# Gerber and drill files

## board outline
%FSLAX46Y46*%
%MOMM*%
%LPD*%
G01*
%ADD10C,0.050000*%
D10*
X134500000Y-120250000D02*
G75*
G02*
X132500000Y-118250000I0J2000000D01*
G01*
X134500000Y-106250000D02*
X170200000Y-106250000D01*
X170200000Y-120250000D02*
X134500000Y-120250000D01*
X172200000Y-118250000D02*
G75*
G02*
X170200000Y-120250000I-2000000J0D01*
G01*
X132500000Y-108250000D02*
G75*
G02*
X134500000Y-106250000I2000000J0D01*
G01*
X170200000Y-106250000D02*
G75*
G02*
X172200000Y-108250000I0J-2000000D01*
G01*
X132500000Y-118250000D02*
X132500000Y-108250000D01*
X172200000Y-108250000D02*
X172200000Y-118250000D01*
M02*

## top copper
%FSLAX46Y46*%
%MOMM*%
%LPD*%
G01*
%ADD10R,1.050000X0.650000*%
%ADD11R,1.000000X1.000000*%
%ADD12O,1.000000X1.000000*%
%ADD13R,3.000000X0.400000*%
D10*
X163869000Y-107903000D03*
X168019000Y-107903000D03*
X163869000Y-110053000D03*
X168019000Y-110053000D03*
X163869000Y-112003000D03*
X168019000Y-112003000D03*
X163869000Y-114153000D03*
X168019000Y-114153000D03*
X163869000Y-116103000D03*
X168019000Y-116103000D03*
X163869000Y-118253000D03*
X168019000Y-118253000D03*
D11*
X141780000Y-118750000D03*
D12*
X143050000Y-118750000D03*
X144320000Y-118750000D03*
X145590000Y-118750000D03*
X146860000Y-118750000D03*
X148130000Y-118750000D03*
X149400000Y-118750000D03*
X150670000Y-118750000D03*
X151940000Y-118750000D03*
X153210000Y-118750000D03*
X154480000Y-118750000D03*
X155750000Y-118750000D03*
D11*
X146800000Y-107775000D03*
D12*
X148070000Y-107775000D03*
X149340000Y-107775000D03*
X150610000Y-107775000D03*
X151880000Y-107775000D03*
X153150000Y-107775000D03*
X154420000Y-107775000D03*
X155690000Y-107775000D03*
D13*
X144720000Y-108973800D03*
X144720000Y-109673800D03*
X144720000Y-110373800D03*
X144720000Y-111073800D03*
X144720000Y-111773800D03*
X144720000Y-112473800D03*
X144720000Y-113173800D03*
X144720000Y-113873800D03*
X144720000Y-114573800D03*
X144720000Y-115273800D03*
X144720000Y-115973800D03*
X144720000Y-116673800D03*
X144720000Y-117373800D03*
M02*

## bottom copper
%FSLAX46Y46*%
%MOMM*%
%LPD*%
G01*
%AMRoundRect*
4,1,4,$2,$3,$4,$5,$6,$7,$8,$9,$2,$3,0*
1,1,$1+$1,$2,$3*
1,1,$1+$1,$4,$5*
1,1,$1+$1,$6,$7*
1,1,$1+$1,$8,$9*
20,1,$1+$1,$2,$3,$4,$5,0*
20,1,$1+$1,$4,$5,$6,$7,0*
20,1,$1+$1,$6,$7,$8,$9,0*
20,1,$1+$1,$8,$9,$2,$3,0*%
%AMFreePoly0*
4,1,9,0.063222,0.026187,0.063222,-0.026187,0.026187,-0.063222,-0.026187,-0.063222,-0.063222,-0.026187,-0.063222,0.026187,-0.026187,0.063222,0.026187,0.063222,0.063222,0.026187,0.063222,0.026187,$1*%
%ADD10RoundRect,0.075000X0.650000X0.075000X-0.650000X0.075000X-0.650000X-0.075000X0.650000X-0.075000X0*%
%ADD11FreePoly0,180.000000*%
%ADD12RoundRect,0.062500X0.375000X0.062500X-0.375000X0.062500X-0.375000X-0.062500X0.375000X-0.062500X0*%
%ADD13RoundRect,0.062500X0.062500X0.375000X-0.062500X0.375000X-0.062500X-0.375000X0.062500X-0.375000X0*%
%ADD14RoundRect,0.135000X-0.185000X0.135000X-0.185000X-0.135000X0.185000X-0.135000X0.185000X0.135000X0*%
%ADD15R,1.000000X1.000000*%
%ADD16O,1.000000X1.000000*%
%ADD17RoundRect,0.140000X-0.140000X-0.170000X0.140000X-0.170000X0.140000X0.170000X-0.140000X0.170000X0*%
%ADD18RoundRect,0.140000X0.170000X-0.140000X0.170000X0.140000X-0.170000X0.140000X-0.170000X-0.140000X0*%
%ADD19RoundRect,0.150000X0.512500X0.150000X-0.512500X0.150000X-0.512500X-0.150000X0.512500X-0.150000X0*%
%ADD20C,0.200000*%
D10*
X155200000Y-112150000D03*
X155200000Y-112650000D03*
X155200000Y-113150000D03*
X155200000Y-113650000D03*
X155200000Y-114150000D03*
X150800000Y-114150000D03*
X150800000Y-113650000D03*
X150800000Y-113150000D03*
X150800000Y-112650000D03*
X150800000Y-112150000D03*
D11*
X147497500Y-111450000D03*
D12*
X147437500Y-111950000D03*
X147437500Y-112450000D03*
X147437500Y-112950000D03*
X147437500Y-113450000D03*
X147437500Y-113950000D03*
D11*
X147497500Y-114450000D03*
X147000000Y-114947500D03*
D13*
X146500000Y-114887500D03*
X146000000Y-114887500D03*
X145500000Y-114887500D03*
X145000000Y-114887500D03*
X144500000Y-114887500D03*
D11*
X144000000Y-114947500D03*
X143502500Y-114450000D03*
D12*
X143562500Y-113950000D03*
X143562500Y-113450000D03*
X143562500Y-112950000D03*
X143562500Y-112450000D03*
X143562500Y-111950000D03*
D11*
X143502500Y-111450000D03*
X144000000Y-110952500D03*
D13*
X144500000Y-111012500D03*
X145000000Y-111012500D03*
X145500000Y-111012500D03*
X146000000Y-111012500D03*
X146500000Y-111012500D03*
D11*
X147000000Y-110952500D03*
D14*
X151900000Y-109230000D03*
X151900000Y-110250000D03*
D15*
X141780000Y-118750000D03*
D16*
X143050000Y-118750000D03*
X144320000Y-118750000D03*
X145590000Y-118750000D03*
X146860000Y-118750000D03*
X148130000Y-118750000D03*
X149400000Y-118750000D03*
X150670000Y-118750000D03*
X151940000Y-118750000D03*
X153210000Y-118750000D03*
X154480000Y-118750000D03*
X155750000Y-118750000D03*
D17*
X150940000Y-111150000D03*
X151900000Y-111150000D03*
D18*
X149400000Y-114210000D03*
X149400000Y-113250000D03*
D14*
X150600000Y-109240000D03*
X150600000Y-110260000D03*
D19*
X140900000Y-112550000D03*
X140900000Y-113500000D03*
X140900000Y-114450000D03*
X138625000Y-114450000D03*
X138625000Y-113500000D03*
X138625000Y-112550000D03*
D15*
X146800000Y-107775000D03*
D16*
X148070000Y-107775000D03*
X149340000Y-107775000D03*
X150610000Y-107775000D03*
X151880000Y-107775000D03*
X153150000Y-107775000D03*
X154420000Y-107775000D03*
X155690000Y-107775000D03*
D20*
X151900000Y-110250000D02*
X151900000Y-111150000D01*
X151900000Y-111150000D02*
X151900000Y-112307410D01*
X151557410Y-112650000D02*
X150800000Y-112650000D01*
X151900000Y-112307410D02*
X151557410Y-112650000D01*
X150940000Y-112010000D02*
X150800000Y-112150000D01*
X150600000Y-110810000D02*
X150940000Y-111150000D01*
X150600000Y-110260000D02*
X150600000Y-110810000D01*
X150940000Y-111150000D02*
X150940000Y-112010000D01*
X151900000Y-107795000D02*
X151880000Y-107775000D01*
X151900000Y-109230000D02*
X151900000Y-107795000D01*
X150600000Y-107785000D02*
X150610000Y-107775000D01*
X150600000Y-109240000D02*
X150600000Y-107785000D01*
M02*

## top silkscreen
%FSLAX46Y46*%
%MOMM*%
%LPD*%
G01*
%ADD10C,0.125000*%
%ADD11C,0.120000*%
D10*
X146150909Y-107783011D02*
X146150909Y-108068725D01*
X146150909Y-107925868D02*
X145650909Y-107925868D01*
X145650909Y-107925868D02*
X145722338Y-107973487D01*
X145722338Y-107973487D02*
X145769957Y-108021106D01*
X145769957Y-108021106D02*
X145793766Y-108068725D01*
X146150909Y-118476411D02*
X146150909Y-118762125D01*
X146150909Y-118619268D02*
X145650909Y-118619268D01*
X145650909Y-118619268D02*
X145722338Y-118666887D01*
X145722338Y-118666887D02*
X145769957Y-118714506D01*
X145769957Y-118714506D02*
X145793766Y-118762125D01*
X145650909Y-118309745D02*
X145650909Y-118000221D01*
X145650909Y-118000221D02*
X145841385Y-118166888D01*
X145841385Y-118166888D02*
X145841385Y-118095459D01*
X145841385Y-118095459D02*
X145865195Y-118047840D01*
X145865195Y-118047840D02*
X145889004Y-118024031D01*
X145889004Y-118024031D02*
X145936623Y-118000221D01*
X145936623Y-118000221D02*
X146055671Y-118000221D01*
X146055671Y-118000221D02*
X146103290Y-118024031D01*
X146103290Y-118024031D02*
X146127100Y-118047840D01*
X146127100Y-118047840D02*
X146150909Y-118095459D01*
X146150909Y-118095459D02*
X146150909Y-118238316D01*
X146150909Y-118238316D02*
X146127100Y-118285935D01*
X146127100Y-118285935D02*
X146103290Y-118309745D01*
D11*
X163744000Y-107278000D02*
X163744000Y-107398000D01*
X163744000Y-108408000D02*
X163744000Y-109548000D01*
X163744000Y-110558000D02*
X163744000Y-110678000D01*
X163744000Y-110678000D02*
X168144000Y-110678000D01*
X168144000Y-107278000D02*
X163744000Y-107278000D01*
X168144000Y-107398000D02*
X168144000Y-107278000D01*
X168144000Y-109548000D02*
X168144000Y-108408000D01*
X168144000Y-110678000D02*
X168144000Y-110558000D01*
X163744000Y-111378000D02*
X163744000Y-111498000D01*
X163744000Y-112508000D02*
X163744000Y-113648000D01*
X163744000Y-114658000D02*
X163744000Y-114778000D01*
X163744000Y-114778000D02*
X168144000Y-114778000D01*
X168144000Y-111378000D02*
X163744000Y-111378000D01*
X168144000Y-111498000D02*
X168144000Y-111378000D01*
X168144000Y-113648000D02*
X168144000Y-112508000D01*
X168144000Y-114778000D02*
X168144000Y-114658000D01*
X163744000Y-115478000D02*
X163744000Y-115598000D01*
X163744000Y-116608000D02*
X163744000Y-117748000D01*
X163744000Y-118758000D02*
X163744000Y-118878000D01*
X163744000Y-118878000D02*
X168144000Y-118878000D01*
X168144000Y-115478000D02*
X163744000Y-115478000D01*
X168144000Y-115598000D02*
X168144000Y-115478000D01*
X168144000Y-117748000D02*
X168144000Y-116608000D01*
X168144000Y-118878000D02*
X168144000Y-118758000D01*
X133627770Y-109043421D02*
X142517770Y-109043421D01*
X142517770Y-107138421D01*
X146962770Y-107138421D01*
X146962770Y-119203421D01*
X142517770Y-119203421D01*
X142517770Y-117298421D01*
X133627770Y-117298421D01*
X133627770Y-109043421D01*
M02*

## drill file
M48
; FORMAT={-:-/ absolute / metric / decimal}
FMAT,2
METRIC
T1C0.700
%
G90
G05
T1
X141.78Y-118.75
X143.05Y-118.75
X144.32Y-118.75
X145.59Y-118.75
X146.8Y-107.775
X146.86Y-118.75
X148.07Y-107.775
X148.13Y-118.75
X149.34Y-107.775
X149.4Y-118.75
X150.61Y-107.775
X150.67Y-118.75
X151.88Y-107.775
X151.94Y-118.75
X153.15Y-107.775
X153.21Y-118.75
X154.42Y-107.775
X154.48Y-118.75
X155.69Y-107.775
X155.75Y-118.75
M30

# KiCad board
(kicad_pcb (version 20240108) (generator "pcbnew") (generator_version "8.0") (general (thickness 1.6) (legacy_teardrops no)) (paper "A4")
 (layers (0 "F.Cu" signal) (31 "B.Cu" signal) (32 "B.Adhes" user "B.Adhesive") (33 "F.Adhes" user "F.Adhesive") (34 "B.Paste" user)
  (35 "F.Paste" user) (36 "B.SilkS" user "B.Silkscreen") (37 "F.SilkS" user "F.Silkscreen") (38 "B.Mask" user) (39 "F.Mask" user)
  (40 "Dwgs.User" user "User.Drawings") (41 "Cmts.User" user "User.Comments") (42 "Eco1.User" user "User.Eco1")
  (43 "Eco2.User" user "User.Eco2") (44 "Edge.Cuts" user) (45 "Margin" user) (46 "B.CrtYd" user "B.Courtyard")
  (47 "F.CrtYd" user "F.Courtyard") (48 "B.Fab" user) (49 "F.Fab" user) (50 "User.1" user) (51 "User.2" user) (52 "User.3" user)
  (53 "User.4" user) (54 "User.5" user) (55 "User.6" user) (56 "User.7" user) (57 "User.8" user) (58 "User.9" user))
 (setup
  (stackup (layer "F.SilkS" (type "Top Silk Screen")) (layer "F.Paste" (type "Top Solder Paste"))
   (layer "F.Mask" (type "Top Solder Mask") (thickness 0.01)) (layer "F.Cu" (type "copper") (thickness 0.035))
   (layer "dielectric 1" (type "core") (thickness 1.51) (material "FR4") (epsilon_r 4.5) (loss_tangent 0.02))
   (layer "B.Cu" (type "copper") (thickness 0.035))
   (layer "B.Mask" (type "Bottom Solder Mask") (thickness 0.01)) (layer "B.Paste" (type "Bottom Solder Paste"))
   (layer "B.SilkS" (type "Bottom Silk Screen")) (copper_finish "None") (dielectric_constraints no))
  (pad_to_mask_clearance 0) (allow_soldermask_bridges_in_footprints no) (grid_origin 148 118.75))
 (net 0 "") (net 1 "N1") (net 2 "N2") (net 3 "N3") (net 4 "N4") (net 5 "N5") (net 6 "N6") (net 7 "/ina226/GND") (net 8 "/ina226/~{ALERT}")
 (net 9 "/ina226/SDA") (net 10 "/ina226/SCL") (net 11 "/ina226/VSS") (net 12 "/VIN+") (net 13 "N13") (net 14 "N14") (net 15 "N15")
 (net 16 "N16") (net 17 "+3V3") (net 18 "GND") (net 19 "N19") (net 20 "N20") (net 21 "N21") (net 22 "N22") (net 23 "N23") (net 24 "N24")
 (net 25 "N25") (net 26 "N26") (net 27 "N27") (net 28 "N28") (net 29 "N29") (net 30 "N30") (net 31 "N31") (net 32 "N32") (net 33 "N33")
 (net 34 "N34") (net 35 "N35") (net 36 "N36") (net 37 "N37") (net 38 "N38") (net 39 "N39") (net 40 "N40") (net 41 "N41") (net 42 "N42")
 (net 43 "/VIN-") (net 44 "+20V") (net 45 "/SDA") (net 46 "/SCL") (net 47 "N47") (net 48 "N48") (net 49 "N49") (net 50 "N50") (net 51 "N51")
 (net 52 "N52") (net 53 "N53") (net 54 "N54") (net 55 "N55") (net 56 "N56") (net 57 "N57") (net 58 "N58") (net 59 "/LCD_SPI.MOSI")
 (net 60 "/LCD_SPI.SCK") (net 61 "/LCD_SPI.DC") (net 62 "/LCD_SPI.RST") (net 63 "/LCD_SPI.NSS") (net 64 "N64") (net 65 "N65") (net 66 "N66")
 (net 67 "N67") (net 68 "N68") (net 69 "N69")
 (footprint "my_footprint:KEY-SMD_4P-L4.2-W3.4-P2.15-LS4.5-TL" (layer "F.Cu") (at 166 109.05)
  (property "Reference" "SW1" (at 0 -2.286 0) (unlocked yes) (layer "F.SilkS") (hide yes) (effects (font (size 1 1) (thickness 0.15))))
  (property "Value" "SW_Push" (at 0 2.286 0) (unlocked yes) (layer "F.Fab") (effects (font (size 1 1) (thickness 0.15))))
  (fp_line (start -2.256 -1.772) (end -2.256 -1.652) (stroke (width 0.12) (type solid)) (layer "F.SilkS"))
  (fp_line (start -2.256 -0.642) (end -2.256 0.498) (stroke (width 0.12) (type solid)) (layer "F.SilkS"))
  (fp_line (start -2.256 1.508) (end -2.256 1.628) (stroke (width 0.12) (type solid)) (layer "F.SilkS"))
  (fp_line (start -2.256 1.628) (end 2.144 1.628) (stroke (width 0.12) (type solid)) (layer "F.SilkS"))
  (fp_line (start 2.144 -1.772) (end -2.256 -1.772) (stroke (width 0.12) (type solid)) (layer "F.SilkS"))
  (fp_line (start 2.144 -1.652) (end 2.144 -1.772) (stroke (width 0.12) (type solid)) (layer "F.SilkS"))
  (fp_line (start 2.144 0.498) (end 2.144 -0.642) (stroke (width 0.12) (type solid)) (layer "F.SilkS"))
  (fp_line (start 2.144 1.628) (end 2.144 1.508) (stroke (width 0.12) (type solid)) (layer "F.SilkS"))
  (pad "1" smd rect (at -2.131 -1.147) (size 1.05 0.65) (layers "F.Cu" "F.Paste" "F.Mask") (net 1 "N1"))
  (pad "1" smd rect (at 2.019 -1.147) (size 1.05 0.65) (layers "F.Cu" "F.Paste" "F.Mask") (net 1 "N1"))
  (pad "2" smd rect (at -2.131 1.003) (size 1.05 0.65) (layers "F.Cu" "F.Paste" "F.Mask") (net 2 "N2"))
  (pad "2" smd rect (at 2.019 1.003) (size 1.05 0.65) (layers "F.Cu" "F.Paste" "F.Mask") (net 2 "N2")))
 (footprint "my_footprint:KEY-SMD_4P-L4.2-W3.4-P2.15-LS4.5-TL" (layer "F.Cu") (at 166 113.15)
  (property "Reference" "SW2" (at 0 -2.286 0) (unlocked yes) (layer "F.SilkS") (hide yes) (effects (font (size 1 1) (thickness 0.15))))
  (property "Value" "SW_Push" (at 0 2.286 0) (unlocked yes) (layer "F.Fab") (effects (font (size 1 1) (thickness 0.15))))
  (fp_line (start -2.256 -1.772) (end -2.256 -1.652) (stroke (width 0.12) (type solid)) (layer "F.SilkS"))
  (fp_line (start -2.256 -0.642) (end -2.256 0.498) (stroke (width 0.12) (type solid)) (layer "F.SilkS"))
  (fp_line (start -2.256 1.508) (end -2.256 1.628) (stroke (width 0.12) (type solid)) (layer "F.SilkS"))
  (fp_line (start -2.256 1.628) (end 2.144 1.628) (stroke (width 0.12) (type solid)) (layer "F.SilkS"))
  (fp_line (start 2.144 -1.772) (end -2.256 -1.772) (stroke (width 0.12) (type solid)) (layer "F.SilkS"))
  (fp_line (start 2.144 -1.652) (end 2.144 -1.772) (stroke (width 0.12) (type solid)) (layer "F.SilkS"))
  (fp_line (start 2.144 0.498) (end 2.144 -0.642) (stroke (width 0.12) (type solid)) (layer "F.SilkS"))
  (fp_line (start 2.144 1.628) (end 2.144 1.508) (stroke (width 0.12) (type solid)) (layer "F.SilkS"))
  (pad "1" smd rect (at -2.131 -1.147) (size 1.05 0.65) (layers "F.Cu" "F.Paste" "F.Mask") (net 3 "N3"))
  (pad "1" smd rect (at 2.019 -1.147) (size 1.05 0.65) (layers "F.Cu" "F.Paste" "F.Mask") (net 3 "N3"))
  (pad "2" smd rect (at -2.131 1.003) (size 1.05 0.65) (layers "F.Cu" "F.Paste" "F.Mask") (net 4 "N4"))
  (pad "2" smd rect (at 2.019 1.003) (size 1.05 0.65) (layers "F.Cu" "F.Paste" "F.Mask") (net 4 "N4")))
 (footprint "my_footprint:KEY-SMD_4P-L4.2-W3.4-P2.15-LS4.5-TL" (layer "F.Cu") (at 166 117.25)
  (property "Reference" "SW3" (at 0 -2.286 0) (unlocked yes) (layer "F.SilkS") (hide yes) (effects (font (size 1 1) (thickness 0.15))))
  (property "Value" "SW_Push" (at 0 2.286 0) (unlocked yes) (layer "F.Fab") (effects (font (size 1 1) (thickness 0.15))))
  (fp_line (start -2.256 -1.772) (end -2.256 -1.652) (stroke (width 0.12) (type solid)) (layer "F.SilkS"))
  (fp_line (start -2.256 -0.642) (end -2.256 0.498) (stroke (width 0.12) (type solid)) (layer "F.SilkS"))
  (fp_line (start -2.256 1.508) (end -2.256 1.628) (stroke (width 0.12) (type solid)) (layer "F.SilkS"))
  (fp_line (start -2.256 1.628) (end 2.144 1.628) (stroke (width 0.12) (type solid)) (layer "F.SilkS"))
  (fp_line (start 2.144 -1.772) (end -2.256 -1.772) (stroke (width 0.12) (type solid)) (layer "F.SilkS"))
  (fp_line (start 2.144 -1.652) (end 2.144 -1.772) (stroke (width 0.12) (type solid)) (layer "F.SilkS"))
  (fp_line (start 2.144 0.498) (end 2.144 -0.642) (stroke (width 0.12) (type solid)) (layer "F.SilkS"))
  (fp_line (start 2.144 1.628) (end 2.144 1.508) (stroke (width 0.12) (type solid)) (layer "F.SilkS"))
  (pad "1" smd rect (at -2.131 -1.147) (size 1.05 0.65) (layers "F.Cu" "F.Paste" "F.Mask") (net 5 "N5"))
  (pad "1" smd rect (at 2.019 -1.147) (size 1.05 0.65) (layers "F.Cu" "F.Paste" "F.Mask") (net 5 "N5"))
  (pad "2" smd rect (at -2.131 1.003) (size 1.05 0.65) (layers "F.Cu" "F.Paste" "F.Mask") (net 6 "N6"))
  (pad "2" smd rect (at 2.019 1.003) (size 1.05 0.65) (layers "F.Cu" "F.Paste" "F.Mask") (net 6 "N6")))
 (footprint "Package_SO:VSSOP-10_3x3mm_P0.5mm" (layer "B.Cu") (at 153 113.15 180)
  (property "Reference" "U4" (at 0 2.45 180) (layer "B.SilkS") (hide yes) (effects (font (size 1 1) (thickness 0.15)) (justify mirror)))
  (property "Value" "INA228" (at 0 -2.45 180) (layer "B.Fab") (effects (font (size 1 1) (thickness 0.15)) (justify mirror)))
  (pad "1" smd roundrect (at -2.2 1 180) (size 1.45 0.3) (layers "B.Cu" "B.Paste" "B.Mask") (roundrect_rratio 0.25) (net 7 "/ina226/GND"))
  (pad "2" smd roundrect (at -2.2 0.5 180) (size 1.45 0.3) (layers "B.Cu" "B.Paste" "B.Mask") (roundrect_rratio 0.25) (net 7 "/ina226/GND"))
  (pad "3" smd roundrect (at -2.2 0 180) (size 1.45 0.3) (layers "B.Cu" "B.Paste" "B.Mask") (roundrect_rratio 0.25)
   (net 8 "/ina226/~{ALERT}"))
  (pad "4" smd roundrect (at -2.2 -0.5 180) (size 1.45 0.3) (layers "B.Cu" "B.Paste" "B.Mask") (roundrect_rratio 0.25) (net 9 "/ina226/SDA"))
  (pad "5" smd roundrect (at -2.2 -1 180) (size 1.45 0.3) (layers "B.Cu" "B.Paste" "B.Mask") (roundrect_rratio 0.25) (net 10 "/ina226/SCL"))
  (pad "6" smd roundrect (at 2.2 -1 180) (size 1.45 0.3) (layers "B.Cu" "B.Paste" "B.Mask") (roundrect_rratio 0.25) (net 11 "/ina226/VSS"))
  (pad "7" smd roundrect (at 2.2 -0.5 180) (size 1.45 0.3) (layers "B.Cu" "B.Paste" "B.Mask") (roundrect_rratio 0.25) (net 7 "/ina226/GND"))
  (pad "8" smd roundrect (at 2.2 0 180) (size 1.45 0.3) (layers "B.Cu" "B.Paste" "B.Mask") (roundrect_rratio 0.25) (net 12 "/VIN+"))
  (pad "9" smd roundrect (at 2.2 0.5 180) (size 1.45 0.3) (layers "B.Cu" "B.Paste" "B.Mask") (roundrect_rratio 0.25) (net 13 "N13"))
  (pad "10" smd roundrect (at 2.2 1 180) (size 1.45 0.3) (layers "B.Cu" "B.Paste" "B.Mask") (roundrect_rratio 0.25) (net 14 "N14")))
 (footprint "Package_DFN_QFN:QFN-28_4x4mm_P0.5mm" (layer "B.Cu") (at 145.5 112.95 180)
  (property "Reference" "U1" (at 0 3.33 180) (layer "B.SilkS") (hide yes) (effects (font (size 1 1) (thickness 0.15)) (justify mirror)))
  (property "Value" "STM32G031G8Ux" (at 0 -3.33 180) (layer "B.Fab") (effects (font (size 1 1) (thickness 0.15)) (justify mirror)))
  (pad "1" smd custom (at -1.9975 1.5 180) (size 0.136863 0.136863) (layers "B.Cu" "B.Paste" "B.Mask") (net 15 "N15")
   (options (clearance outline) (anchor circle)) (primitives))
  (pad "2" smd roundrect (at -1.9375 1 180) (size 0.875 0.25) (layers "B.Cu" "B.Paste" "B.Mask") (roundrect_rratio 0.25) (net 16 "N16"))
  (pad "3" smd roundrect (at -1.9375 0.5 180) (size 0.875 0.25) (layers "B.Cu" "B.Paste" "B.Mask") (roundrect_rratio 0.25) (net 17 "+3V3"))
  (pad "4" smd roundrect (at -1.9375 0 180) (size 0.875 0.25) (layers "B.Cu" "B.Paste" "B.Mask") (roundrect_rratio 0.25) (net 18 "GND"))
  (pad "5" smd roundrect (at -1.9375 -0.5 180) (size 0.875 0.25) (layers "B.Cu" "B.Paste" "B.Mask") (roundrect_rratio 0.25) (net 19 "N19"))
  (pad "6" smd roundrect (at -1.9375 -1 180) (size 0.875 0.25) (layers "B.Cu" "B.Paste" "B.Mask") (roundrect_rratio 0.25) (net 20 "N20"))
  (pad "7" smd custom (at -1.9975 -1.5 180) (size 0.136863 0.136863) (layers "B.Cu" "B.Paste" "B.Mask") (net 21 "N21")
   (options (clearance outline) (anchor circle)) (primitives))
  (pad "8" smd custom (at -1.5 -1.9975 180) (size 0.136863 0.136863) (layers "B.Cu" "B.Paste" "B.Mask") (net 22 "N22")
   (options (clearance outline) (anchor circle)) (primitives))
  (pad "9" smd roundrect (at -1 -1.9375 180) (size 0.25 0.875) (layers "B.Cu" "B.Paste" "B.Mask") (roundrect_rratio 0.25) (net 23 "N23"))
  (pad "10" smd roundrect (at -0.5 -1.9375 180) (size 0.25 0.875) (layers "B.Cu" "B.Paste" "B.Mask") (roundrect_rratio 0.25) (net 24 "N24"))
  (pad "11" smd roundrect (at 0 -1.9375 180) (size 0.25 0.875) (layers "B.Cu" "B.Paste" "B.Mask") (roundrect_rratio 0.25) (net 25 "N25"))
  (pad "12" smd roundrect (at 0.5 -1.9375 180) (size 0.25 0.875) (layers "B.Cu" "B.Paste" "B.Mask") (roundrect_rratio 0.25) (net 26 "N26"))
  (pad "13" smd roundrect (at 1 -1.9375 180) (size 0.25 0.875) (layers "B.Cu" "B.Paste" "B.Mask") (roundrect_rratio 0.25) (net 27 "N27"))
  (pad "14" smd custom (at 1.5 -1.9975 180) (size 0.136863 0.136863) (layers "B.Cu" "B.Paste" "B.Mask") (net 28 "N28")
   (options (clearance outline) (anchor circle)) (primitives))
  (pad "15" smd custom (at 1.9975 -1.5 180) (size 0.136863 0.136863) (layers "B.Cu" "B.Paste" "B.Mask") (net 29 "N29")
   (options (clearance outline) (anchor circle)) (primitives))
  (pad "16" smd roundrect (at 1.9375 -1 180) (size 0.875 0.25) (layers "B.Cu" "B.Paste" "B.Mask") (roundrect_rratio 0.25) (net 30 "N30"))
  (pad "17" smd roundrect (at 1.9375 -0.5 180) (size 0.875 0.25) (layers "B.Cu" "B.Paste" "B.Mask") (roundrect_rratio 0.25) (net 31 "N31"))
  (pad "18" smd roundrect (at 1.9375 0 180) (size 0.875 0.25) (layers "B.Cu" "B.Paste" "B.Mask") (roundrect_rratio 0.25) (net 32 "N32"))
  (pad "19" smd roundrect (at 1.9375 0.5 180) (size 0.875 0.25) (layers "B.Cu" "B.Paste" "B.Mask") (roundrect_rratio 0.25) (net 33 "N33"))
  (pad "20" smd roundrect (at 1.9375 1 180) (size 0.875 0.25) (layers "B.Cu" "B.Paste" "B.Mask") (roundrect_rratio 0.25) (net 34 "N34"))
  (pad "21" smd custom (at 1.9975 1.5 180) (size 0.136863 0.136863) (layers "B.Cu" "B.Paste" "B.Mask") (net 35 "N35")
   (options (clearance outline) (anchor circle)) (primitives))
  (pad "22" smd custom (at 1.5 1.9975 180) (size 0.136863 0.136863) (layers "B.Cu" "B.Paste" "B.Mask") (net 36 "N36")
   (options (clearance outline) (anchor circle)) (primitives))
  (pad "23" smd roundrect (at 1 1.9375 180) (size 0.25 0.875) (layers "B.Cu" "B.Paste" "B.Mask") (roundrect_rratio 0.25) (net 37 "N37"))
  (pad "24" smd roundrect (at 0.5 1.9375 180) (size 0.25 0.875) (layers "B.Cu" "B.Paste" "B.Mask") (roundrect_rratio 0.25) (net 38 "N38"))
  (pad "25" smd roundrect (at 0 1.9375 180) (size 0.25 0.875) (layers "B.Cu" "B.Paste" "B.Mask") (roundrect_rratio 0.25) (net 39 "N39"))
  (pad "26" smd roundrect (at -0.5 1.9375 180) (size 0.25 0.875) (layers "B.Cu" "B.Paste" "B.Mask") (roundrect_rratio 0.25) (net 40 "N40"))
  (pad "27" smd roundrect (at -1 1.9375 180) (size 0.25 0.875) (layers "B.Cu" "B.Paste" "B.Mask") (roundrect_rratio 0.25) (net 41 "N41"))
  (pad "28" smd custom (at -1.5 1.9975 180) (size 0.136863 0.136863) (layers "B.Cu" "B.Paste" "B.Mask") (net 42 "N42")
   (options (clearance outline) (anchor circle)) (primitives)))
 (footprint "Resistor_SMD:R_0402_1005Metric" (layer "B.Cu") (at 151.9 109.74 -90)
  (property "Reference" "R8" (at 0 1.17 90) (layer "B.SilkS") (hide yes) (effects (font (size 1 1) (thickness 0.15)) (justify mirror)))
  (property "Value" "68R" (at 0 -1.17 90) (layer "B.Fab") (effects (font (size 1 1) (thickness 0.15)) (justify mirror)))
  (pad "1" smd roundrect (at -0.51 0 270) (size 0.54 0.64) (layers "B.Cu" "B.Paste" "B.Mask") (roundrect_rratio 0.25) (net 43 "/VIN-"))
  (pad "2" smd roundrect (at 0.51 0 270) (size 0.54 0.64) (layers "B.Cu" "B.Paste" "B.Mask") (roundrect_rratio 0.25) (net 13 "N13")))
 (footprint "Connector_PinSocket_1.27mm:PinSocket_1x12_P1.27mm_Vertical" (layer "B.Cu") (at 141.78 118.75 -90)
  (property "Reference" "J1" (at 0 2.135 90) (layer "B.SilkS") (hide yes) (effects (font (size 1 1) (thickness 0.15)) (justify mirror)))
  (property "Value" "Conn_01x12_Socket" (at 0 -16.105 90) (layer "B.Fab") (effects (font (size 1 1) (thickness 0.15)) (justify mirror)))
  (pad "1" thru_hole rect (at 0 0 270) (size 1 1) (drill 0.7) (layers "*.Cu" "*.Mask") (remove_unused_layers no) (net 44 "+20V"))
  (pad "2" thru_hole oval (at 0 -1.27 270) (size 1 1) (drill 0.7) (layers "*.Cu" "*.Mask") (remove_unused_layers no) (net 44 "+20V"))
  (pad "3" thru_hole oval (at 0 -2.54 270) (size 1 1) (drill 0.7) (layers "*.Cu" "*.Mask") (remove_unused_layers no) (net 44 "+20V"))
  (pad "4" thru_hole oval (at 0 -3.81 270) (size 1 1) (drill 0.7) (layers "*.Cu" "*.Mask") (remove_unused_layers no) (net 44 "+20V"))
  (pad "5" thru_hole oval (at 0 -5.08 270) (size 1 1) (drill 0.7) (layers "*.Cu" "*.Mask") (remove_unused_layers no) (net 44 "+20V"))
  (pad "6" thru_hole oval (at 0 -6.35 270) (size 1 1) (drill 0.7) (layers "*.Cu" "*.Mask") (remove_unused_layers no) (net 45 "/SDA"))
  (pad "7" thru_hole oval (at 0 -7.62 270) (size 1 1) (drill 0.7) (layers "*.Cu" "*.Mask") (remove_unused_layers no) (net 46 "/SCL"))
  (pad "8" thru_hole oval (at 0 -8.89 270) (size 1 1) (drill 0.7) (layers "*.Cu" "*.Mask") (remove_unused_layers no) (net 18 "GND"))
  (pad "9" thru_hole oval (at 0 -10.16 270) (size 1 1) (drill 0.7) (layers "*.Cu" "*.Mask") (remove_unused_layers no) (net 18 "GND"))
  (pad "10" thru_hole oval (at 0 -11.43 270) (size 1 1) (drill 0.7) (layers "*.Cu" "*.Mask") (remove_unused_layers no) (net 18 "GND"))
  (pad "11" thru_hole oval (at 0 -12.7 270) (size 1 1) (drill 0.7) (layers "*.Cu" "*.Mask") (remove_unused_layers no) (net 18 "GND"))
  (pad "12" thru_hole oval (at 0 -13.97 270) (size 1 1) (drill 0.7) (layers "*.Cu" "*.Mask") (remove_unused_layers no) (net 18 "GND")))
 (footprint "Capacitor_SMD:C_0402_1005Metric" (layer "B.Cu") (at 151.42 111.15)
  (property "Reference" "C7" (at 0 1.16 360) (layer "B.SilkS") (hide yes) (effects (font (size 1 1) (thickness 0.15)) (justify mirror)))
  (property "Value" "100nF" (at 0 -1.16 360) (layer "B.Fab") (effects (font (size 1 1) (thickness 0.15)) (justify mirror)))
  (pad "1" smd roundrect (at -0.48 0) (size 0.56 0.62) (layers "B.Cu" "B.Paste" "B.Mask") (roundrect_rratio 0.25) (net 14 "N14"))
  (pad "2" smd roundrect (at 0.48 0) (size 0.56 0.62) (layers "B.Cu" "B.Paste" "B.Mask") (roundrect_rratio 0.25) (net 13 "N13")))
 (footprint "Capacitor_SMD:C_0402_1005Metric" (layer "B.Cu") (at 149.4 113.73 90)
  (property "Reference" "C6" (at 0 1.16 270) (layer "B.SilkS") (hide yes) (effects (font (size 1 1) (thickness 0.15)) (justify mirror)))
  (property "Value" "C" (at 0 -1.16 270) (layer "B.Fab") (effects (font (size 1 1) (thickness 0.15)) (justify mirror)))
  (pad "1" smd roundrect (at -0.48 0 90) (size 0.56 0.62) (layers "B.Cu" "B.Paste" "B.Mask") (roundrect_rratio 0.25) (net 11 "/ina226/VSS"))
  (pad "2" smd roundrect (at 0.48 0 90) (size 0.56 0.62) (layers "B.Cu" "B.Paste" "B.Mask") (roundrect_rratio 0.25) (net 7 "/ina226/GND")))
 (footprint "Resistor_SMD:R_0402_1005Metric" (layer "B.Cu") (at 150.6 109.75 -90)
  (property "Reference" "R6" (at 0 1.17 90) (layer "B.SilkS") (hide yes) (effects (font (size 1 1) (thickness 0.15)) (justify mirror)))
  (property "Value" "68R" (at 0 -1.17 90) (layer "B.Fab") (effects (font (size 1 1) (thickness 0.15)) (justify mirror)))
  (pad "1" smd roundrect (at -0.51 0 270) (size 0.54 0.64) (layers "B.Cu" "B.Paste" "B.Mask") (roundrect_rratio 0.25) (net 12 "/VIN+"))
  (pad "2" smd roundrect (at 0.51 0 270) (size 0.54 0.64) (layers "B.Cu" "B.Paste" "B.Mask") (roundrect_rratio 0.25) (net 14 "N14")))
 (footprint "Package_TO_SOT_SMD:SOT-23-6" (layer "B.Cu") (at 139.7625 113.5 180)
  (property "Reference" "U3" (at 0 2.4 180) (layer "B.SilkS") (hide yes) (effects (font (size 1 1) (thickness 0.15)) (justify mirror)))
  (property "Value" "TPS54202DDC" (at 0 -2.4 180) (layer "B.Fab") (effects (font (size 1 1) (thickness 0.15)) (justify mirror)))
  (pad "1" smd roundrect (at -1.1375 0.95 180) (size 1.325 0.6) (layers "B.Cu" "B.Paste" "B.Mask") (roundrect_rratio 0.25) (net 18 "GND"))
  (pad "2" smd roundrect (at -1.1375 0 180) (size 1.325 0.6) (layers "B.Cu" "B.Paste" "B.Mask") (roundrect_rratio 0.25) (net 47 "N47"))
  (pad "3" smd roundrect (at -1.1375 -0.95 180) (size 1.325 0.6) (layers "B.Cu" "B.Paste" "B.Mask") (roundrect_rratio 0.25) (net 44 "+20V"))
  (pad "4" smd roundrect (at 1.1375 -0.95 180) (size 1.325 0.6) (layers "B.Cu" "B.Paste" "B.Mask") (roundrect_rratio 0.25) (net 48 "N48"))
  (pad "5" smd roundrect (at 1.1375 0 180) (size 1.325 0.6) (layers "B.Cu" "B.Paste" "B.Mask") (roundrect_rratio 0.25) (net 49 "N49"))
  (pad "6" smd roundrect (at 1.1375 0.95 180) (size 1.325 0.6) (layers "B.Cu" "B.Paste" "B.Mask") (roundrect_rratio 0.25) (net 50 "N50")))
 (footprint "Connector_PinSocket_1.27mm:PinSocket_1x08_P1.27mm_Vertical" (layer "B.Cu") (at 146.8 107.775 -90)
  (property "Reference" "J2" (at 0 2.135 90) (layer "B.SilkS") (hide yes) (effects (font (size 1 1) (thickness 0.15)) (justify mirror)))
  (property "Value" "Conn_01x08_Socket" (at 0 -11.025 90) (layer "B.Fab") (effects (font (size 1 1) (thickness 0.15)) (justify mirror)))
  (pad "1" thru_hole rect (at 0 0 270) (size 1 1) (drill 0.7) (layers "*.Cu" "*.Mask") (remove_unused_layers no) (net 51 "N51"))
  (pad "2" thru_hole oval (at 0 -1.27 270) (size 1 1) (drill 0.7) (layers "*.Cu" "*.Mask") (remove_unused_layers no) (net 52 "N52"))
  (pad "3" thru_hole oval (at 0 -2.54 270) (size 1 1) (drill 0.7) (layers "*.Cu" "*.Mask") (remove_unused_layers no) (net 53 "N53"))
  (pad "4" thru_hole oval (at 0 -3.81 270) (size 1 1) (drill 0.7) (layers "*.Cu" "*.Mask") (remove_unused_layers no) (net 12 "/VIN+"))
  (pad "5" thru_hole oval (at 0 -5.08 270) (size 1 1) (drill 0.7) (layers "*.Cu" "*.Mask") (remove_unused_layers no) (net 43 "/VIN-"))
  (pad "6" thru_hole oval (at 0 -6.35 270) (size 1 1) (drill 0.7) (layers "*.Cu" "*.Mask") (remove_unused_layers no) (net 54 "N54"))
  (pad "7" thru_hole oval (at 0 -7.62 270) (size 1 1) (drill 0.7) (layers "*.Cu" "*.Mask") (remove_unused_layers no) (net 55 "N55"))
  (pad "8" thru_hole oval (at 0 -8.89 270) (size 1 1) (drill 0.7) (layers "*.Cu" "*.Mask") (remove_unused_layers no) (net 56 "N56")))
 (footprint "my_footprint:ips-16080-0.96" (layer "B.Cu") (at 149.8 113.25 180)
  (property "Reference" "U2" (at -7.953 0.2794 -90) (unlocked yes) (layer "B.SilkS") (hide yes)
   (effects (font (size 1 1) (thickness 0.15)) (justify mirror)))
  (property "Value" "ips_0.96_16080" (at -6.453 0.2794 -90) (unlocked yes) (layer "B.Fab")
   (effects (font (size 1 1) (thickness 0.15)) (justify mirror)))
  (fp_poly
   (pts (xy 16.17223 4.206579) (xy 7.28223 4.206579) (xy 7.28223 6.111579) (xy 2.83723 6.111579) (xy 2.83723 -5.953421)
    (xy 7.28223 -5.953421) (xy 7.28223 -4.048421) (xy 16.17223 -4.048421))
   (stroke (width 0.12) (type solid)) (fill none) (layer "F.SilkS"))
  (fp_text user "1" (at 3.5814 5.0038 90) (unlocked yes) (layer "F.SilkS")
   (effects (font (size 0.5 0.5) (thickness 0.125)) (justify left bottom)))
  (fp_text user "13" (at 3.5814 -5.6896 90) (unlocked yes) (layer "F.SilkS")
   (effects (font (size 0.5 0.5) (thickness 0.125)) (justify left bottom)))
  (pad "1" smd rect (at 5.08 4.2762 180) (size 3 0.4) (layers "F.Cu" "F.Paste" "F.Mask") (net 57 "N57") (zone_connect 0)
   (thermal_bridge_angle 45))
  (pad "2" smd rect (at 5.08 3.5762 180) (size 3 0.4) (layers "F.Cu" "F.Paste" "F.Mask") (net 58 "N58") (zone_connect 0)
   (thermal_bridge_angle 45))
  (pad "3" smd rect (at 5.08 2.8762 180) (size 3 0.4) (layers "F.Cu" "F.Paste" "F.Mask") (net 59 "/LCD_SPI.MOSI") (zone_connect 0)
   (thermal_bridge_angle 45))
  (pad "4" smd rect (at 5.08 2.1762 180) (size 3 0.4) (layers "F.Cu" "F.Paste" "F.Mask") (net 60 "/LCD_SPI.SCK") (zone_connect 0)
   (thermal_bridge_angle 45))
  (pad "5" smd rect (at 5.08 1.4762 180) (size 3 0.4) (layers "F.Cu" "F.Paste" "F.Mask") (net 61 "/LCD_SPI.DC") (zone_connect 0)
   (thermal_bridge_angle 45))
  (pad "6" smd rect (at 5.08 0.7762 180) (size 3 0.4) (layers "F.Cu" "F.Paste" "F.Mask") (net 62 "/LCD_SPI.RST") (zone_connect 0)
   (thermal_bridge_angle 45))
  (pad "7" smd rect (at 5.08 0.0762 180) (size 3 0.4) (layers "F.Cu" "F.Paste" "F.Mask") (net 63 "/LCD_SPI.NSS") (zone_connect 0)
   (thermal_bridge_angle 45))
  (pad "8" smd rect (at 5.08 -0.6238 180) (size 3 0.4) (layers "F.Cu" "F.Paste" "F.Mask") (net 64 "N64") (zone_connect 0)
   (thermal_bridge_angle 45))
  (pad "9" smd rect (at 5.08 -1.3238 180) (size 3 0.4) (layers "F.Cu" "F.Paste" "F.Mask") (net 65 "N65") (zone_connect 0)
   (thermal_bridge_angle 45))
  (pad "10" smd rect (at 5.08 -2.0238 180) (size 3 0.4) (layers "F.Cu" "F.Paste" "F.Mask") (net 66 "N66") (zone_connect 0)
   (thermal_bridge_angle 45))
  (pad "11" smd rect (at 5.08 -2.7238 180) (size 3 0.4) (layers "F.Cu" "F.Paste" "F.Mask") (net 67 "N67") (zone_connect 0)
   (thermal_bridge_angle 45))
  (pad "12" smd rect (at 5.08 -3.4238 180) (size 3 0.4) (layers "F.Cu" "F.Paste" "F.Mask") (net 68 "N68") (zone_connect 0)
   (thermal_bridge_angle 45))
  (pad "13" smd rect (at 5.08 -4.1238 180) (size 3 0.4) (layers "F.Cu" "F.Paste" "F.Mask") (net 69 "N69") (zone_connect 0)
   (thermal_bridge_angle 45)))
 (gr_arc (start 134.5 120.25) (mid 133.085786 119.664214) (end 132.5 118.25) (stroke (width 0.05) (type default)) (layer "Edge.Cuts"))
 (gr_line (start 134.5 106.25) (end 170.2 106.25) (stroke (width 0.05) (type default)) (layer "Edge.Cuts"))
 (gr_line (start 170.2 120.25) (end 134.5 120.25) (stroke (width 0.05) (type default)) (layer "Edge.Cuts"))
 (gr_arc (start 172.2 118.25) (mid 171.614214 119.664214) (end 170.2 120.25) (stroke (width 0.05) (type default)) (layer "Edge.Cuts"))
 (gr_arc (start 132.5 108.25) (mid 133.085786 106.835786) (end 134.5 106.25) (stroke (width 0.05) (type default)) (layer "Edge.Cuts"))
 (gr_arc (start 170.2 106.25) (mid 171.614214 106.835786) (end 172.2 108.25) (stroke (width 0.05) (type default)) (layer "Edge.Cuts"))
 (gr_line (start 132.5 118.25) (end 132.5 108.25) (stroke (width 0.05) (type default)) (layer "Edge.Cuts"))
 (gr_line (start 172.2 108.25) (end 172.2 118.25) (stroke (width 0.05) (type default)) (layer "Edge.Cuts"))
 (segment (start 151.9 110.25) (end 151.9 111.15) (width 0.2) (layer "B.Cu") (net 13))
 (segment (start 151.9 111.15) (end 151.9 112.30741) (width 0.2) (layer "B.Cu") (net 13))
 (segment (start 151.55741 112.65) (end 150.8 112.65) (width 0.2) (layer "B.Cu") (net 13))
 (segment (start 151.9 112.30741) (end 151.55741 112.65) (width 0.2) (layer "B.Cu") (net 13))
 (segment (start 150.94 112.01) (end 150.8 112.15) (width 0.2) (layer "B.Cu") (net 14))
 (segment (start 150.6 110.81) (end 150.94 111.15) (width 0.2) (layer "B.Cu") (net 14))
 (segment (start 150.6 110.26) (end 150.6 110.81) (width 0.2) (layer "B.Cu") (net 14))
 (segment (start 150.94 111.15) (end 150.94 112.01) (width 0.2) (layer "B.Cu") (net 14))
 (segment (start 151.9 107.795) (end 151.88 107.775) (width 0.2) (layer "B.Cu") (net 43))
 (segment (start 151.9 109.23) (end 151.9 107.795) (width 0.2) (layer "B.Cu") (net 43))
 (segment (start 150.6 107.785) (end 150.61 107.775) (width 0.2) (layer "B.Cu") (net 12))
 (segment (start 150.6 109.24) (end 150.6 107.785) (width 0.2) (layer "B.Cu") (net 12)))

